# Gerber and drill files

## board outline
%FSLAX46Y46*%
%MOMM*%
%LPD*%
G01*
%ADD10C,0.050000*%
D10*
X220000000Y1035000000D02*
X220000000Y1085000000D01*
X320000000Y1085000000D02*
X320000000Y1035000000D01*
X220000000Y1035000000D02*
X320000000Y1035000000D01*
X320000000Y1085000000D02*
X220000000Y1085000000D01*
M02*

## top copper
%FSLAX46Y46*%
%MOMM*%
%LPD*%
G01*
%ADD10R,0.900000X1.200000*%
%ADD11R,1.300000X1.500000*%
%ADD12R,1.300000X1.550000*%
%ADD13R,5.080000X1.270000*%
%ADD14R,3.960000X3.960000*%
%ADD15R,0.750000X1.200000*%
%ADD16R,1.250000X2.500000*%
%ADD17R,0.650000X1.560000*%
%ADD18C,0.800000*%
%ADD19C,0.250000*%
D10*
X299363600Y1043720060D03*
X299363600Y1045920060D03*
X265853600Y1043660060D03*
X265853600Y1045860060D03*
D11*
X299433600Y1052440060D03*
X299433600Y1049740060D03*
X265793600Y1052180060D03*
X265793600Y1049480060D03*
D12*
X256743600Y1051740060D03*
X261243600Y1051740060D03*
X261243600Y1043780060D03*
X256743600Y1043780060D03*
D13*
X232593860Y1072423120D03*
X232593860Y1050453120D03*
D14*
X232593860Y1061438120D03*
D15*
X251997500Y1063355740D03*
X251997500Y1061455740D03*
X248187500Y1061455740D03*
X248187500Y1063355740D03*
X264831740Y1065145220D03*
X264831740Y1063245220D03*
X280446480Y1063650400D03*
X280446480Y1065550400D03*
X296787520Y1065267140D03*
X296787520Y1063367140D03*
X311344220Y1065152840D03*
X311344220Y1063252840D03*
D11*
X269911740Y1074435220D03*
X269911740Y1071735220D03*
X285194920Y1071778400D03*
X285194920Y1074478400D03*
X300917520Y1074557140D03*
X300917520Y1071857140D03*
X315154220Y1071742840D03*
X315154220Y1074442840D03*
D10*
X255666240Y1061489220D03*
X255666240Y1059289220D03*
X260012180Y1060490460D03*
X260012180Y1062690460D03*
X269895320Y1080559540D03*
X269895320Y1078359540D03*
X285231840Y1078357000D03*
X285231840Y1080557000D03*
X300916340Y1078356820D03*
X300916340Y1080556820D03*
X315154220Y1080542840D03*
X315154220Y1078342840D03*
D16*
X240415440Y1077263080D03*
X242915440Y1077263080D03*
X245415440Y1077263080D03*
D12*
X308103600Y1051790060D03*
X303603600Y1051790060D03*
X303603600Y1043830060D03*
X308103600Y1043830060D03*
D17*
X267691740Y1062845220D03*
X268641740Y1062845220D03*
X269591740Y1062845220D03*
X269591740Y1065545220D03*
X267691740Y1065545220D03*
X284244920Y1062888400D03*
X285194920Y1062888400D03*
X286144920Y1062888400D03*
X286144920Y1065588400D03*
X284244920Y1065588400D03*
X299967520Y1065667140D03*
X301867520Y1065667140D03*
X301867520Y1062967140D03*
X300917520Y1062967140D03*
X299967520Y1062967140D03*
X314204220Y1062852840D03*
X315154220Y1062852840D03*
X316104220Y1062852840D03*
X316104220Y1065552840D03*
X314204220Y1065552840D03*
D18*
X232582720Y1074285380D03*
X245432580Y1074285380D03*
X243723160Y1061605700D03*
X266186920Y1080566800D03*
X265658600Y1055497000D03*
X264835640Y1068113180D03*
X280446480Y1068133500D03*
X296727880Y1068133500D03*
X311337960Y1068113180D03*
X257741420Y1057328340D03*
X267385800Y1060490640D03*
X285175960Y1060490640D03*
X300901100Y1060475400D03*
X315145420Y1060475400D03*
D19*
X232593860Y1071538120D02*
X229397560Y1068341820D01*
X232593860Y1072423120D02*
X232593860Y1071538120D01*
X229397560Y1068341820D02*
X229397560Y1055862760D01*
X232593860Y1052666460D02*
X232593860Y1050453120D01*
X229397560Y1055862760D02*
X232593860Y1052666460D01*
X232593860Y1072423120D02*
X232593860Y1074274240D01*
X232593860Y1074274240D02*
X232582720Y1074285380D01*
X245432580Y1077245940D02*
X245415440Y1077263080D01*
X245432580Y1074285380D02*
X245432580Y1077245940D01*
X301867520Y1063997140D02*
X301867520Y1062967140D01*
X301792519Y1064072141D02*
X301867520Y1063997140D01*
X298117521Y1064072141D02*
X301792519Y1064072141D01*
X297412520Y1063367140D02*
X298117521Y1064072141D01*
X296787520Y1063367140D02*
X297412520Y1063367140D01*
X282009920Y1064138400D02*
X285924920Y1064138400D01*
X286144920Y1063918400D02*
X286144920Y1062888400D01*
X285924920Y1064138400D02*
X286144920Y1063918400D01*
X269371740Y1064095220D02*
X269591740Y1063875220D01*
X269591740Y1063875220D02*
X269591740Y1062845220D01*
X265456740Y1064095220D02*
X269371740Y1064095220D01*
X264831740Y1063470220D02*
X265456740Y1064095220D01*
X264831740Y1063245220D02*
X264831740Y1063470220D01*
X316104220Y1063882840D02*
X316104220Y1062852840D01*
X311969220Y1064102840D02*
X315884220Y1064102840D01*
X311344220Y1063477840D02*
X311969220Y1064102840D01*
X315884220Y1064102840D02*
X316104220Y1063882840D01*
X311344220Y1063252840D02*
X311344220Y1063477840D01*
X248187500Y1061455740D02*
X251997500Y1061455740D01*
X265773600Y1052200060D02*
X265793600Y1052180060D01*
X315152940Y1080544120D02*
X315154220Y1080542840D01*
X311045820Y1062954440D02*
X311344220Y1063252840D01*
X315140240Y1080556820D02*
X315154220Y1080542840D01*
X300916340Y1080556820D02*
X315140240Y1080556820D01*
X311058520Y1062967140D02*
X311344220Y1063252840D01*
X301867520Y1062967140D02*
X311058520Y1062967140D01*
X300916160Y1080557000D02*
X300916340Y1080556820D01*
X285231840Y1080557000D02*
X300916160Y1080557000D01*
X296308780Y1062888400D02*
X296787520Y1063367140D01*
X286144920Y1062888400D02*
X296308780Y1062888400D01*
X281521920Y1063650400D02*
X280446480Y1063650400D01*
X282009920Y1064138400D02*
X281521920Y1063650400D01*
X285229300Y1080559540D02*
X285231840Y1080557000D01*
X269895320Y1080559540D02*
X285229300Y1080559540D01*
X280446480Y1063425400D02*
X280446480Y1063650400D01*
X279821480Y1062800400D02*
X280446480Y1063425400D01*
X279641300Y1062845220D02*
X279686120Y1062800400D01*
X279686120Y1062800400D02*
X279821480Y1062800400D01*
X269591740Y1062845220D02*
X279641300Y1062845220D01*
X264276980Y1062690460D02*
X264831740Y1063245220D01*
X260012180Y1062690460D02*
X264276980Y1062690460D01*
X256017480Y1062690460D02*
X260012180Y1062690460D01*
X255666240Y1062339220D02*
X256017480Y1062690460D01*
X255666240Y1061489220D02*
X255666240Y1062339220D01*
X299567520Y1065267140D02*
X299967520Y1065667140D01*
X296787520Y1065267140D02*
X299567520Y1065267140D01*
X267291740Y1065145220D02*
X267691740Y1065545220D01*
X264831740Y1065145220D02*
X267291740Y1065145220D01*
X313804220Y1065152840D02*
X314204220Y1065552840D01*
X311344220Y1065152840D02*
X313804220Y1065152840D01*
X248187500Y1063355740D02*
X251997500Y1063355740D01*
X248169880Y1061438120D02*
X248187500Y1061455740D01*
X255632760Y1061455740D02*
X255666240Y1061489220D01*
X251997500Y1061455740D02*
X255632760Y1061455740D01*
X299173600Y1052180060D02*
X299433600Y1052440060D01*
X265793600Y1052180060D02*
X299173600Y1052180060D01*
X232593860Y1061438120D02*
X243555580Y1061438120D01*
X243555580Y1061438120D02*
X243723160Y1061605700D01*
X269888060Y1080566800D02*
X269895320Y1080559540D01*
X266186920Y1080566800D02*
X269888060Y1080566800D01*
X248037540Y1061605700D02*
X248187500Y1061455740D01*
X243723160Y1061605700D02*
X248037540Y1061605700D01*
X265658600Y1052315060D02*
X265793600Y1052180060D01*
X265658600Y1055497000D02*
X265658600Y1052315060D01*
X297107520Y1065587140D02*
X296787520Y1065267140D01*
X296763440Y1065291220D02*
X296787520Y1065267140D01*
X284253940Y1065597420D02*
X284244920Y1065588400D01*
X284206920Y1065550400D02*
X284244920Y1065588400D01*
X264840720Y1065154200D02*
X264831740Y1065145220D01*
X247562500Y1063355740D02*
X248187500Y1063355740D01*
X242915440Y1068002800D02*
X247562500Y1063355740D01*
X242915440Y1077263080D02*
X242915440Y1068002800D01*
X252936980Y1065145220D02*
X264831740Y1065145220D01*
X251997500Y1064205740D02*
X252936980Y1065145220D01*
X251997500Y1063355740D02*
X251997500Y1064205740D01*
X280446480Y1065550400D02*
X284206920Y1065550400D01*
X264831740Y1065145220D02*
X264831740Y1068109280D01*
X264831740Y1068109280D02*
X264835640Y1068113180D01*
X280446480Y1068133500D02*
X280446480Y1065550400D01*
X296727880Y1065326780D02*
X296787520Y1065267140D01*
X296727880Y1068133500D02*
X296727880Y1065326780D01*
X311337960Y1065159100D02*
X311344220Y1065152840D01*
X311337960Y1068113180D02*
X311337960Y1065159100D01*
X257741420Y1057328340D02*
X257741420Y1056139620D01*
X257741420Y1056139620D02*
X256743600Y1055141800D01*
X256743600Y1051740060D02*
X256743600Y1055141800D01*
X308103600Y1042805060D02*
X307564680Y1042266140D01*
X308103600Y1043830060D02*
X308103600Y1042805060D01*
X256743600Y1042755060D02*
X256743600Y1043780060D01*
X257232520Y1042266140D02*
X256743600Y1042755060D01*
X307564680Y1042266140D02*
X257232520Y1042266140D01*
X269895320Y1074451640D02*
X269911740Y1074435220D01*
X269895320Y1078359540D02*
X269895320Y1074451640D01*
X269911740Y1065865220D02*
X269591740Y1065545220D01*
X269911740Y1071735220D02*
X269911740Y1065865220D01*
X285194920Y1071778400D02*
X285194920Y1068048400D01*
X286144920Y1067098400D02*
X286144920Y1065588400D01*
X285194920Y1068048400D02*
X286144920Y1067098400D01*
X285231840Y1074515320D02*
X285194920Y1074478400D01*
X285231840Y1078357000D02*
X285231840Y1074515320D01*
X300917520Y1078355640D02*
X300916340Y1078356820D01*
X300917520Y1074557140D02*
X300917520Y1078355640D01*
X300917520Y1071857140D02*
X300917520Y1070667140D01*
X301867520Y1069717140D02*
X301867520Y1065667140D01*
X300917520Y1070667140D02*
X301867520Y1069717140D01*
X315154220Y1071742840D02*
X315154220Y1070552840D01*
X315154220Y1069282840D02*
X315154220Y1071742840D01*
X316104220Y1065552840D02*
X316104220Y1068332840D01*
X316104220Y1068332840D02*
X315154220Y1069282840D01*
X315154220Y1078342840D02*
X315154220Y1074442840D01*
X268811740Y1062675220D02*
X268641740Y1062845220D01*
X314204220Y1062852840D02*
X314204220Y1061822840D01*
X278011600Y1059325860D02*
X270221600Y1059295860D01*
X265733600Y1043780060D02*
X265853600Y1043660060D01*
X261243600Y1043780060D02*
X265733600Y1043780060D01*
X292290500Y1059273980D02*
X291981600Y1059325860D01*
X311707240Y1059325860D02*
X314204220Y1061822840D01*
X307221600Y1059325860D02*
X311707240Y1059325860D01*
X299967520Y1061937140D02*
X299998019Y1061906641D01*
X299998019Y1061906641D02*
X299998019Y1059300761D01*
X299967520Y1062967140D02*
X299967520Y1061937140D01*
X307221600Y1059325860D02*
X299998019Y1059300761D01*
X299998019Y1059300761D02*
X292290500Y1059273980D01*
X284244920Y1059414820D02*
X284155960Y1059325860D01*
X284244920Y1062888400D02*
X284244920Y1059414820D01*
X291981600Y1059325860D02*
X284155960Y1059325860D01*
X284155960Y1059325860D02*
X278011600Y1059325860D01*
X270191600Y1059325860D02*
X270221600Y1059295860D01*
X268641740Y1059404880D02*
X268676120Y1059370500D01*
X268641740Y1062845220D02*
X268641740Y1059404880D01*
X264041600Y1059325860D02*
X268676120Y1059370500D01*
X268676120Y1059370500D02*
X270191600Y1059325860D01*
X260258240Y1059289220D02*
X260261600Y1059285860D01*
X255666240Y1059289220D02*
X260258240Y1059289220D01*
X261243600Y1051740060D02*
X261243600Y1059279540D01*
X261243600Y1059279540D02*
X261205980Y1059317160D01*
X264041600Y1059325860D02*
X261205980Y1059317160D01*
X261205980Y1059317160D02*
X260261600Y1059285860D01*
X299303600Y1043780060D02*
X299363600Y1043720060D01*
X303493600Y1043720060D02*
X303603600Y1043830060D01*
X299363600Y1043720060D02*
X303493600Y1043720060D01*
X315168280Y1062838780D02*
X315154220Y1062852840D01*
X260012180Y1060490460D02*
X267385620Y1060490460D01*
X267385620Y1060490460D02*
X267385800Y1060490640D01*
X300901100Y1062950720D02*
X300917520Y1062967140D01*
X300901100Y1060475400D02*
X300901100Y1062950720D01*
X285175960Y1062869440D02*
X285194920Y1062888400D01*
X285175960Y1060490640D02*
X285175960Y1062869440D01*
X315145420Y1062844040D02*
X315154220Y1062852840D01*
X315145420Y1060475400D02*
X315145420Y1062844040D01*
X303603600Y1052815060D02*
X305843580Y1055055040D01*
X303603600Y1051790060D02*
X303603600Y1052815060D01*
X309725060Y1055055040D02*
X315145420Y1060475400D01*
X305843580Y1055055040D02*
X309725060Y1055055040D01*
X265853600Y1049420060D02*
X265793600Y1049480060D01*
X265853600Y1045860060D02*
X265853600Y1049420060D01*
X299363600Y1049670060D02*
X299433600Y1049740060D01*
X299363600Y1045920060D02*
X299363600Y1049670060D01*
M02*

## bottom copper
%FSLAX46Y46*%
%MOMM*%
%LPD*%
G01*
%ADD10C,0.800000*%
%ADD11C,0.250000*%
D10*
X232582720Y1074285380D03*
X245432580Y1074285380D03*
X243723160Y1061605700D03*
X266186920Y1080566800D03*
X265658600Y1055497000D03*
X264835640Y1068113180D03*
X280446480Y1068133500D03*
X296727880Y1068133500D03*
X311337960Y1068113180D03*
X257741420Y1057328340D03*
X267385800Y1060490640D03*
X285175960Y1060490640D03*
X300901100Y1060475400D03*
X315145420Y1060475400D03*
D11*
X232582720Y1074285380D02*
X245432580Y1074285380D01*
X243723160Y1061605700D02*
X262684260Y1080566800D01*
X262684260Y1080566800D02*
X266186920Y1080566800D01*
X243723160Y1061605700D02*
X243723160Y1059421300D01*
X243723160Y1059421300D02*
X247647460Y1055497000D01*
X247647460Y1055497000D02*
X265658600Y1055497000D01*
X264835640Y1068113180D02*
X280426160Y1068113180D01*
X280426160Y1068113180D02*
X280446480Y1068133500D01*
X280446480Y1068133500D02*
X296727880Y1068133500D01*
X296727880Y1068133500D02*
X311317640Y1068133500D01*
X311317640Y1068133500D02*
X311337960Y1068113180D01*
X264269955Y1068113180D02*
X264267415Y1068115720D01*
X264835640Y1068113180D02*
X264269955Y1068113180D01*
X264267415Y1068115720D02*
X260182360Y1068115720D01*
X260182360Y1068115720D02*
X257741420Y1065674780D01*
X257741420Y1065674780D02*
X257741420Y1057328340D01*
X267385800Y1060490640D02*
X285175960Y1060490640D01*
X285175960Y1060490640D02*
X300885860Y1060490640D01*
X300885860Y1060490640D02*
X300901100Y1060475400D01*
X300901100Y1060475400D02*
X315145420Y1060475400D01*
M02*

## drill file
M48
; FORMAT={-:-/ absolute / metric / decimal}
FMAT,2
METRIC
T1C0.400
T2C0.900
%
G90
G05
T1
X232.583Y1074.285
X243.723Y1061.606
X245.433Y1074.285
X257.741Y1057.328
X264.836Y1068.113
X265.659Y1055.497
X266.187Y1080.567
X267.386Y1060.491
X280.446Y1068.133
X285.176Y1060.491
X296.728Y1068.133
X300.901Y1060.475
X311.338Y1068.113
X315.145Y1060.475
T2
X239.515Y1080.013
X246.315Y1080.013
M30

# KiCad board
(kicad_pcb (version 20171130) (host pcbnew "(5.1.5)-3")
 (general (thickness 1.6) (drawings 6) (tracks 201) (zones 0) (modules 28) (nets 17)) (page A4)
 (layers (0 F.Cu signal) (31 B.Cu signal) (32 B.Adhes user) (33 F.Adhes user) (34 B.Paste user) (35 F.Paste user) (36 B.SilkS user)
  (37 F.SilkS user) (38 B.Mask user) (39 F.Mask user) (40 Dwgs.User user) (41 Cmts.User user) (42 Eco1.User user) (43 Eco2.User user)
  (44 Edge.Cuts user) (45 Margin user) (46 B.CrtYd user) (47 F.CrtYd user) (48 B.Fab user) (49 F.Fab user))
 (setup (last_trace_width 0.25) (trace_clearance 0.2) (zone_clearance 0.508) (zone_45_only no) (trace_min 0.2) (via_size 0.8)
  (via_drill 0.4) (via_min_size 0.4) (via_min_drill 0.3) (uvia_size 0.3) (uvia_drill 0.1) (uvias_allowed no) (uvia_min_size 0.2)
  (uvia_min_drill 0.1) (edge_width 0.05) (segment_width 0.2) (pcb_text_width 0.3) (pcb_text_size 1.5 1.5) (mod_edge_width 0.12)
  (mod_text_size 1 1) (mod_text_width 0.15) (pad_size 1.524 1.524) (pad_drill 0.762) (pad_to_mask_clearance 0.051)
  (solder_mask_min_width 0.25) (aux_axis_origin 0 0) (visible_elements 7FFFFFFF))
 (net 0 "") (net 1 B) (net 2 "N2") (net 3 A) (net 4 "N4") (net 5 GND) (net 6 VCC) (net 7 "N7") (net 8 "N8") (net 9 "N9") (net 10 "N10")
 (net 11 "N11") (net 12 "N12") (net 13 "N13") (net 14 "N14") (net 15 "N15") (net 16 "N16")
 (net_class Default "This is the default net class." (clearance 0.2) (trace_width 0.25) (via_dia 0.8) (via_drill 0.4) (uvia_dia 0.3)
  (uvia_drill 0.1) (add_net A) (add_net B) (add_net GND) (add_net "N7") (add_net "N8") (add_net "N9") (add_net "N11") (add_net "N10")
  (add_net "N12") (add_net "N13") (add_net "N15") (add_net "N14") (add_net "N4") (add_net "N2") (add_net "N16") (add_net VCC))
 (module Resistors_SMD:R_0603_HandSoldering (layer F.Cu) (at 299.3636 -1044.82006 90)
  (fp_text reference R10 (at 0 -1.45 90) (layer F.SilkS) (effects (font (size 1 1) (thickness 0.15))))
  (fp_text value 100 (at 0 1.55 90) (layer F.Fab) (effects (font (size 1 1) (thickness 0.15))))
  (pad 1 smd rect (at -1.1 0 90) (size 1.2 0.9) (layers F.Cu F.Paste F.Mask) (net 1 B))
  (pad 2 smd rect (at 1.1 0 90) (size 1.2 0.9) (layers F.Cu F.Paste F.Mask) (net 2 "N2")))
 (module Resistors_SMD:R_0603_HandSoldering (layer F.Cu) (at 265.8536 -1044.76006 90)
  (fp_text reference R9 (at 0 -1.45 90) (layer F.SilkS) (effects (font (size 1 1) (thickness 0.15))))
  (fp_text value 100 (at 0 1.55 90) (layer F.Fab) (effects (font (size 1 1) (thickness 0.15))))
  (pad 1 smd rect (at -1.1 0 90) (size 1.2 0.9) (layers F.Cu F.Paste F.Mask) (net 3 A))
  (pad 2 smd rect (at 1.1 0 90) (size 1.2 0.9) (layers F.Cu F.Paste F.Mask) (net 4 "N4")))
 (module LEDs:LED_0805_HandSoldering (layer F.Cu) (at 299.4336 -1051.09006 270)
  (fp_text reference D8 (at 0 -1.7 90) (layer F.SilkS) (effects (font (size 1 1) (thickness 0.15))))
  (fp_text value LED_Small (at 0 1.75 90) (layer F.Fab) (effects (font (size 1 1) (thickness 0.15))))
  (pad 1 smd rect (at -1.35 0 270) (size 1.5 1.3) (layers F.Cu F.Paste F.Mask) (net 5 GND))
  (pad 2 smd rect (at 1.35 0 270) (size 1.5 1.3) (layers F.Cu F.Paste F.Mask) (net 2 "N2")))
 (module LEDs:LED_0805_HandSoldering (layer F.Cu) (at 265.7936 -1050.83006 270)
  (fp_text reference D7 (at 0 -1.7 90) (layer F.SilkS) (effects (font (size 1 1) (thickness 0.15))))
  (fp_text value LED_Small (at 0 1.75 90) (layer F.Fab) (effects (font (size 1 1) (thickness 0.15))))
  (pad 1 smd rect (at -1.35 0 270) (size 1.5 1.3) (layers F.Cu F.Paste F.Mask) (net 5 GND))
  (pad 2 smd rect (at 1.35 0 270) (size 1.5 1.3) (layers F.Cu F.Paste F.Mask) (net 4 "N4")))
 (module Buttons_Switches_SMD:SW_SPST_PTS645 (layer F.Cu) (at 258.9936 -1047.76006 270)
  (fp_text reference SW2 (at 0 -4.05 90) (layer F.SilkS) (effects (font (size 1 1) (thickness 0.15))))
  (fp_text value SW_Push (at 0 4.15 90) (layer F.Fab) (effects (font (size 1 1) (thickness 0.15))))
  (pad 2 smd rect (at -3.98 2.25 270) (size 1.55 1.3) (layers F.Cu F.Paste F.Mask) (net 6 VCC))
  (pad 1 smd rect (at -3.98 -2.25 270) (size 1.55 1.3) (layers F.Cu F.Paste F.Mask) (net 3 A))
  (pad 1 smd rect (at 3.98 -2.25 270) (size 1.55 1.3) (layers F.Cu F.Paste F.Mask) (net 3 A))
  (pad 2 smd rect (at 3.98 2.25 270) (size 1.55 1.3) (layers F.Cu F.Paste F.Mask) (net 6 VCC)))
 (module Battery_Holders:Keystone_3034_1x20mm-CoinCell (layer F.Cu) (at 232.59386 -1061.43812 270)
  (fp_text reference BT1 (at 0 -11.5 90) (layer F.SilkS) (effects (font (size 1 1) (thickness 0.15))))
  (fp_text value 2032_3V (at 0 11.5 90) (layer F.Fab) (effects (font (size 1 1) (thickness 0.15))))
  (pad 1 smd rect (at -10.985 0 270) (size 1.27 5.08) (layers F.Cu F.Paste F.Mask) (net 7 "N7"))
  (pad 1 smd rect (at 10.985 0 270) (size 1.27 5.08) (layers F.Cu F.Paste F.Mask) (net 7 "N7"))
  (pad 2 smd rect (at 0 0 270) (size 3.96 3.96) (layers F.Cu F.Paste F.Mask) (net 5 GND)))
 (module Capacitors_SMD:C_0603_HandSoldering (layer F.Cu) (at 251.9975 -1062.40574 270)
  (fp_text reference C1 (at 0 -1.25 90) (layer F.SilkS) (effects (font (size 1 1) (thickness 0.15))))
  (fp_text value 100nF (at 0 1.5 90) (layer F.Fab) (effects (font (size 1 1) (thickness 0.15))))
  (pad 1 smd rect (at -0.95 0 270) (size 1.2 0.75) (layers F.Cu F.Paste F.Mask) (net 6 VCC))
  (pad 2 smd rect (at 0.95 0 270) (size 1.2 0.75) (layers F.Cu F.Paste F.Mask) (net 5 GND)))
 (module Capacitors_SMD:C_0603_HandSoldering (layer F.Cu) (at 248.1875 -1062.40574 270)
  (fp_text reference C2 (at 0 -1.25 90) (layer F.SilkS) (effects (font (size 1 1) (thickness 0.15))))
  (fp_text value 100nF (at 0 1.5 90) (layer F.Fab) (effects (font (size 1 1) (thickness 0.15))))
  (pad 2 smd rect (at 0.95 0 270) (size 1.2 0.75) (layers F.Cu F.Paste F.Mask) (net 5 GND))
  (pad 1 smd rect (at -0.95 0 270) (size 1.2 0.75) (layers F.Cu F.Paste F.Mask) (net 6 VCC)))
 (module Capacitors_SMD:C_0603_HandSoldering (layer F.Cu) (at 264.83174 -1064.19522 270)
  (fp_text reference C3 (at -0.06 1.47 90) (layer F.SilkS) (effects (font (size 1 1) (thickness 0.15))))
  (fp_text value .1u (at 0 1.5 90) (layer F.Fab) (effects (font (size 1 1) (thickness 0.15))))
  (pad 1 smd rect (at -0.95 0 270) (size 1.2 0.75) (layers F.Cu F.Paste F.Mask) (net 6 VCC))
  (pad 2 smd rect (at 0.95 0 270) (size 1.2 0.75) (layers F.Cu F.Paste F.Mask) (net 5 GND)))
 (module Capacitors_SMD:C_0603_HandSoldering (layer F.Cu) (at 280.44648 -1064.6004 270)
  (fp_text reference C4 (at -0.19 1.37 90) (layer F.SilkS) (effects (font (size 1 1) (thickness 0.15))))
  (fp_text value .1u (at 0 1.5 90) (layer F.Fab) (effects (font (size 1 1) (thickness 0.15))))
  (pad 2 smd rect (at 0.95 0 270) (size 1.2 0.75) (layers F.Cu F.Paste F.Mask) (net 5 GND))
  (pad 1 smd rect (at -0.95 0 270) (size 1.2 0.75) (layers F.Cu F.Paste F.Mask) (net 6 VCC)))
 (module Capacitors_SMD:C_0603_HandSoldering (layer F.Cu) (at 296.78752 -1064.31714 270)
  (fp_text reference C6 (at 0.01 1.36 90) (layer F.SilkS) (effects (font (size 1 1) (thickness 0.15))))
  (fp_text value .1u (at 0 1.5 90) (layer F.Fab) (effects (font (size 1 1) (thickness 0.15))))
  (pad 1 smd rect (at -0.95 0 270) (size 1.2 0.75) (layers F.Cu F.Paste F.Mask) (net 6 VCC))
  (pad 2 smd rect (at 0.95 0 270) (size 1.2 0.75) (layers F.Cu F.Paste F.Mask) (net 5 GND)))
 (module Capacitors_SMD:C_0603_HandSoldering (layer F.Cu) (at 311.34422 -1064.20284 270)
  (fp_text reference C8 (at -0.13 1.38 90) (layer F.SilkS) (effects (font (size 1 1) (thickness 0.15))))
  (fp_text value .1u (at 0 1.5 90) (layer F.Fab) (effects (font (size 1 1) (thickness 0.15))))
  (pad 1 smd rect (at -0.95 0 270) (size 1.2 0.75) (layers F.Cu F.Paste F.Mask) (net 6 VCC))
  (pad 2 smd rect (at 0.95 0 270) (size 1.2 0.75) (layers F.Cu F.Paste F.Mask) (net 5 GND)))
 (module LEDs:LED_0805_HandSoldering (layer F.Cu) (at 269.91174 -1073.08522 270)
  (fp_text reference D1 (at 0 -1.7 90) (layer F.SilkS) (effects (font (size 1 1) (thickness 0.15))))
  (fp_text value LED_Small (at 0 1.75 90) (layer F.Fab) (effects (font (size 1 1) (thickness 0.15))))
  (pad 1 smd rect (at -1.35 0 270) (size 1.5 1.3) (layers F.Cu F.Paste F.Mask) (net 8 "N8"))
  (pad 2 smd rect (at 1.35 0 270) (size 1.5 1.3) (layers F.Cu F.Paste F.Mask) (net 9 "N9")))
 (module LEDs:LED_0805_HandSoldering (layer F.Cu) (at 285.19492 -1073.1284 270)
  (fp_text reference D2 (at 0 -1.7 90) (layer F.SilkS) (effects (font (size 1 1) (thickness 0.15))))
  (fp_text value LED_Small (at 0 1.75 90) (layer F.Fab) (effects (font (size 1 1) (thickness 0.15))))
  (pad 2 smd rect (at 1.35 0 270) (size 1.5 1.3) (layers F.Cu F.Paste F.Mask) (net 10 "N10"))
  (pad 1 smd rect (at -1.35 0 270) (size 1.5 1.3) (layers F.Cu F.Paste F.Mask) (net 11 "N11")))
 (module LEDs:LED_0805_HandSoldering (layer F.Cu) (at 300.91752 -1073.20714 270)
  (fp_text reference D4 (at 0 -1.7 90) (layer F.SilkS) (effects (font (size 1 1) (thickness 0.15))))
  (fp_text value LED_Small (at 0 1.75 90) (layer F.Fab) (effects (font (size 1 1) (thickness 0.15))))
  (pad 1 smd rect (at -1.35 0 270) (size 1.5 1.3) (layers F.Cu F.Paste F.Mask) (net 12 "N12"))
  (pad 2 smd rect (at 1.35 0 270) (size 1.5 1.3) (layers F.Cu F.Paste F.Mask) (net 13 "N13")))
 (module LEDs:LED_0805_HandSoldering (layer F.Cu) (at 315.15422 -1073.09284 270)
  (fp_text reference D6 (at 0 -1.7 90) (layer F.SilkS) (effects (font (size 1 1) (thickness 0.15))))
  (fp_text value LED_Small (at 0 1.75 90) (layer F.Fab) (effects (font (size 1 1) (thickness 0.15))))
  (pad 2 smd rect (at 1.35 0 270) (size 1.5 1.3) (layers F.Cu F.Paste F.Mask) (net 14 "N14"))
  (pad 1 smd rect (at -1.35 0 270) (size 1.5 1.3) (layers F.Cu F.Paste F.Mask) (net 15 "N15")))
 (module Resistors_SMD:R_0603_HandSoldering (layer F.Cu) (at 255.66624 -1060.38922 270)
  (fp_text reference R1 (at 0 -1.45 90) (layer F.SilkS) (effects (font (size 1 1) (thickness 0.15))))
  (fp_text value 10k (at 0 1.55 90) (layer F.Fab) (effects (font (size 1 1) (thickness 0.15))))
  (pad 1 smd rect (at -1.1 0 270) (size 1.2 0.9) (layers F.Cu F.Paste F.Mask) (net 5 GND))
  (pad 2 smd rect (at 1.1 0 270) (size 1.2 0.9) (layers F.Cu F.Paste F.Mask) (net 3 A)))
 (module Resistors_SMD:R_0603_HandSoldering (layer F.Cu) (at 260.01218 -1061.59046 90)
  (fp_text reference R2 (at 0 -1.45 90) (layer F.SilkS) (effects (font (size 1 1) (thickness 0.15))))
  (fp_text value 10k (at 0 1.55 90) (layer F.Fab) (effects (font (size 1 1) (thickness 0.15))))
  (pad 1 smd rect (at -1.1 0 90) (size 1.2 0.9) (layers F.Cu F.Paste F.Mask) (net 1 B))
  (pad 2 smd rect (at 1.1 0 90) (size 1.2 0.9) (layers F.Cu F.Paste F.Mask) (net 5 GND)))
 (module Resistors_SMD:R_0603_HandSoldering (layer F.Cu) (at 269.89532 -1079.45954 270)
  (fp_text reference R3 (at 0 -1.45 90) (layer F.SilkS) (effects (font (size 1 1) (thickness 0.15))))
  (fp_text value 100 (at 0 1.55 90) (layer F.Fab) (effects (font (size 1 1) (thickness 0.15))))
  (pad 1 smd rect (at -1.1 0 270) (size 1.2 0.9) (layers F.Cu F.Paste F.Mask) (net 5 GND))
  (pad 2 smd rect (at 1.1 0 270) (size 1.2 0.9) (layers F.Cu F.Paste F.Mask) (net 8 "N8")))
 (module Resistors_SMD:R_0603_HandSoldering (layer F.Cu) (at 285.23184 -1079.457 270)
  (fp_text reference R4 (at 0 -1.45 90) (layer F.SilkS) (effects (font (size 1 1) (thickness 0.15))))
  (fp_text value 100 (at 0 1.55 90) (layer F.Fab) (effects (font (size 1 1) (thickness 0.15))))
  (pad 2 smd rect (at 1.1 0 270) (size 1.2 0.9) (layers F.Cu F.Paste F.Mask) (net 11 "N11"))
  (pad 1 smd rect (at -1.1 0 270) (size 1.2 0.9) (layers F.Cu F.Paste F.Mask) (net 5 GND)))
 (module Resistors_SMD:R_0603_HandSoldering (layer F.Cu) (at 300.91634 -1079.45682 270)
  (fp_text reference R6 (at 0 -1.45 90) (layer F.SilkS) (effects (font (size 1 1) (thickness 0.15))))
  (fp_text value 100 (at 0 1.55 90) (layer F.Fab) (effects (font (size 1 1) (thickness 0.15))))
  (pad 2 smd rect (at 1.1 0 270) (size 1.2 0.9) (layers F.Cu F.Paste F.Mask) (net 12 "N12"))
  (pad 1 smd rect (at -1.1 0 270) (size 1.2 0.9) (layers F.Cu F.Paste F.Mask) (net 5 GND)))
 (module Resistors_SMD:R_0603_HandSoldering (layer F.Cu) (at 315.15422 -1079.44284 270)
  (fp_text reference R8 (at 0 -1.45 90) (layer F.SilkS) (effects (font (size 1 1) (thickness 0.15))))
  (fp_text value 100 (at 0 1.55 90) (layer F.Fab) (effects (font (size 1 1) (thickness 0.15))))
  (pad 1 smd rect (at -1.1 0 270) (size 1.2 0.9) (layers F.Cu F.Paste F.Mask) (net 5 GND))
  (pad 2 smd rect (at 1.1 0 270) (size 1.2 0.9) (layers F.Cu F.Paste F.Mask) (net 15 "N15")))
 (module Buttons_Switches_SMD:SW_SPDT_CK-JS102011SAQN (layer F.Cu) (at 242.91544 -1080.01308 180)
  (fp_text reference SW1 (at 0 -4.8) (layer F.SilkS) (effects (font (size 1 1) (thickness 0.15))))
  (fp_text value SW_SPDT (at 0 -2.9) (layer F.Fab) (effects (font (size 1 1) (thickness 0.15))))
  (pad "" np_thru_hole circle (at 3.4 0 180) (size 0.9 0.9) (drill 0.9) (layers *.Cu *.Mask))
  (pad "" np_thru_hole circle (at -3.4 0 180) (size 0.9 0.9) (drill 0.9) (layers *.Cu *.Mask))
  (pad 3 smd rect (at 2.5 -2.75 180) (size 1.25 2.5) (layers F.Cu F.Paste F.Mask) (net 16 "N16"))
  (pad 2 smd rect (at 0 -2.75 180) (size 1.25 2.5) (layers F.Cu F.Paste F.Mask) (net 6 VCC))
  (pad 1 smd rect (at -2.5 -2.75 180) (size 1.25 2.5) (layers F.Cu F.Paste F.Mask) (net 7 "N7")))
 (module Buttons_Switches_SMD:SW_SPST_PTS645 (layer F.Cu) (at 305.8536 -1047.81006 90)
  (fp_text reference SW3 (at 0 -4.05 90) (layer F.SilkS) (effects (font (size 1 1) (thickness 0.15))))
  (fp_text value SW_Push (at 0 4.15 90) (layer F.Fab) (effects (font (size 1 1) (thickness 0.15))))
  (pad 2 smd rect (at 3.98 2.25 90) (size 1.55 1.3) (layers F.Cu F.Paste F.Mask) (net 6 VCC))
  (pad 1 smd rect (at 3.98 -2.25 90) (size 1.55 1.3) (layers F.Cu F.Paste F.Mask) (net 1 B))
  (pad 1 smd rect (at -3.98 -2.25 90) (size 1.55 1.3) (layers F.Cu F.Paste F.Mask) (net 1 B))
  (pad 2 smd rect (at -3.98 2.25 90) (size 1.55 1.3) (layers F.Cu F.Paste F.Mask) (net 6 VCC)))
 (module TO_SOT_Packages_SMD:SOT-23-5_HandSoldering (layer F.Cu) (at 268.64174 -1064.19522 90)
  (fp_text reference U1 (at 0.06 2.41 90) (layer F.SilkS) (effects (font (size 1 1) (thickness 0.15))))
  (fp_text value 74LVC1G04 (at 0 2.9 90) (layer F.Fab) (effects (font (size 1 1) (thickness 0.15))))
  (pad 1 smd rect (at -1.35 -0.95 90) (size 1.56 0.65) (layers F.Cu F.Paste F.Mask))
  (pad 2 smd rect (at -1.35 0 90) (size 1.56 0.65) (layers F.Cu F.Paste F.Mask) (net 3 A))
  (pad 3 smd rect (at -1.35 0.95 90) (size 1.56 0.65) (layers F.Cu F.Paste F.Mask) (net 5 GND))
  (pad 4 smd rect (at 1.35 0.95 90) (size 1.56 0.65) (layers F.Cu F.Paste F.Mask) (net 9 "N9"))
  (pad 5 smd rect (at 1.35 -0.95 90) (size 1.56 0.65) (layers F.Cu F.Paste F.Mask) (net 6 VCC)))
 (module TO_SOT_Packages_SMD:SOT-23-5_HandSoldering (layer F.Cu) (at 285.19492 -1064.2384 90)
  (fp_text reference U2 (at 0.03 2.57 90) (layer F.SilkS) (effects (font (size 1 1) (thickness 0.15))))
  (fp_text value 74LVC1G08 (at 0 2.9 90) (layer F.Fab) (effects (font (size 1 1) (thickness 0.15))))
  (pad 1 smd rect (at -1.35 -0.95 90) (size 1.56 0.65) (layers F.Cu F.Paste F.Mask) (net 3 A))
  (pad 2 smd rect (at -1.35 0 90) (size 1.56 0.65) (layers F.Cu F.Paste F.Mask) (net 1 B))
  (pad 3 smd rect (at -1.35 0.95 90) (size 1.56 0.65) (layers F.Cu F.Paste F.Mask) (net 5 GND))
  (pad 4 smd rect (at 1.35 0.95 90) (size 1.56 0.65) (layers F.Cu F.Paste F.Mask) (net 10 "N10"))
  (pad 5 smd rect (at 1.35 -0.95 90) (size 1.56 0.65) (layers F.Cu F.Paste F.Mask) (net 6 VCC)))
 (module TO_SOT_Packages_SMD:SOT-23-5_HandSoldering (layer F.Cu) (at 300.91752 -1064.31714 90)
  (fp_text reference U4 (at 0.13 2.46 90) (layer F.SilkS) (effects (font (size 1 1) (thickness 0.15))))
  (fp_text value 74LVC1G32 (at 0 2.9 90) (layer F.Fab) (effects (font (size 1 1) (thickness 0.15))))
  (pad 5 smd rect (at 1.35 -0.95 90) (size 1.56 0.65) (layers F.Cu F.Paste F.Mask) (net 6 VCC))
  (pad 4 smd rect (at 1.35 0.95 90) (size 1.56 0.65) (layers F.Cu F.Paste F.Mask) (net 13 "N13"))
  (pad 3 smd rect (at -1.35 0.95 90) (size 1.56 0.65) (layers F.Cu F.Paste F.Mask) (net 5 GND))
  (pad 2 smd rect (at -1.35 0 90) (size 1.56 0.65) (layers F.Cu F.Paste F.Mask) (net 1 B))
  (pad 1 smd rect (at -1.35 -0.95 90) (size 1.56 0.65) (layers F.Cu F.Paste F.Mask) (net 3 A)))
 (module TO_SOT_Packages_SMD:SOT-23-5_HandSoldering (layer F.Cu) (at 315.15422 -1064.20284 90)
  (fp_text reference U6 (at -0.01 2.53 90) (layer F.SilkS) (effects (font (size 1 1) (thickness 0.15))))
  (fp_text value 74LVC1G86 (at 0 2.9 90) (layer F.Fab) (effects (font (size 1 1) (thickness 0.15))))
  (pad 1 smd rect (at -1.35 -0.95 90) (size 1.56 0.65) (layers F.Cu F.Paste F.Mask) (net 3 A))
  (pad 2 smd rect (at -1.35 0 90) (size 1.56 0.65) (layers F.Cu F.Paste F.Mask) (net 1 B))
  (pad 3 smd rect (at -1.35 0.95 90) (size 1.56 0.65) (layers F.Cu F.Paste F.Mask) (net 5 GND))
  (pad 4 smd rect (at 1.35 0.95 90) (size 1.56 0.65) (layers F.Cu F.Paste F.Mask) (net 14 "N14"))
  (pad 5 smd rect (at 1.35 -0.95 90) (size 1.56 0.65) (layers F.Cu F.Paste F.Mask) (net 6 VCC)))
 (gr_line (start 220 -1035) (end 220 -1085) (layer Edge.Cuts) (width 0.05))
 (gr_line (start 320 -1085) (end 320 -1035) (layer Edge.Cuts) (width 0.05))
 (gr_line (start 220 -1035) (end 320 -1035) (layer Edge.Cuts) (width 0.05))
 (gr_line (start 320 -1085) (end 220 -1085) (layer Edge.Cuts) (width 0.05))
 (segment (start 232.59386 -1071.53812) (end 229.39756 -1068.34182) (width 0.25) (layer F.Cu) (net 7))
 (segment (start 232.59386 -1072.42312) (end 232.59386 -1071.53812) (width 0.25) (layer F.Cu) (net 7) (status 10))
 (segment (start 229.39756 -1068.34182) (end 229.39756 -1055.86276) (width 0.25) (layer F.Cu) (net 7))
 (segment (start 232.59386 -1052.66646) (end 232.59386 -1050.45312) (width 0.25) (layer F.Cu) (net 7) (status 20))
 (segment (start 229.39756 -1055.86276) (end 232.59386 -1052.66646) (width 0.25) (layer F.Cu) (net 7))
 (via (at 232.58272 -1074.28538) (size 0.8) (drill 0.4) (layers F.Cu B.Cu) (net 7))
 (segment (start 232.59386 -1072.42312) (end 232.59386 -1074.27424) (width 0.25) (layer F.Cu) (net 7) (status 10))
 (segment (start 232.59386 -1074.27424) (end 232.58272 -1074.28538) (width 0.25) (layer F.Cu) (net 7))
 (via (at 245.43258 -1074.28538) (size 0.8) (drill 0.4) (layers F.Cu B.Cu) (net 7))
 (segment (start 232.58272 -1074.28538) (end 245.43258 -1074.28538) (width 0.25) (layer B.Cu) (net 7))
 (segment (start 245.43258 -1077.24594) (end 245.41544 -1077.26308) (width 0.25) (layer F.Cu) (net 7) (status 30))
 (segment (start 245.43258 -1074.28538) (end 245.43258 -1077.24594) (width 0.25) (layer F.Cu) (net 7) (status 20))
 (segment (start 301.86752 -1063.99714) (end 301.86752 -1062.96714) (width 0.25) (layer F.Cu) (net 5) (status 20))
 (segment (start 301.792519 -1064.072141) (end 301.86752 -1063.99714) (width 0.25) (layer F.Cu) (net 5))
 (segment (start 298.117521 -1064.072141) (end 301.792519 -1064.072141) (width 0.25) (layer F.Cu) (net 5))
 (segment (start 297.41252 -1063.36714) (end 298.117521 -1064.072141) (width 0.25) (layer F.Cu) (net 5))
 (segment (start 296.78752 -1063.36714) (end 297.41252 -1063.36714) (width 0.25) (layer F.Cu) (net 5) (status 10))
 (segment (start 282.00992 -1064.1384) (end 285.92492 -1064.1384) (width 0.25) (layer F.Cu) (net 5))
 (segment (start 286.14492 -1063.9184) (end 286.14492 -1062.8884) (width 0.25) (layer F.Cu) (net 5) (status 20))
 (segment (start 285.92492 -1064.1384) (end 286.14492 -1063.9184) (width 0.25) (layer F.Cu) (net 5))
 (segment (start 269.37174 -1064.09522) (end 269.59174 -1063.87522) (width 0.25) (layer F.Cu) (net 5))
 (segment (start 269.59174 -1063.87522) (end 269.59174 -1062.84522) (width 0.25) (layer F.Cu) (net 5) (status 20))
 (segment (start 265.45674 -1064.09522) (end 269.37174 -1064.09522) (width 0.25) (layer F.Cu) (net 5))
 (segment (start 264.83174 -1063.47022) (end 265.45674 -1064.09522) (width 0.25) (layer F.Cu) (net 5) (status 10))
 (segment (start 264.83174 -1063.24522) (end 264.83174 -1063.47022) (width 0.25) (layer F.Cu) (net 5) (status 30))
 (segment (start 316.10422 -1063.88284) (end 316.10422 -1062.85284) (width 0.25) (layer F.Cu) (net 5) (status 20))
 (segment (start 311.96922 -1064.10284) (end 315.88422 -1064.10284) (width 0.25) (layer F.Cu) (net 5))
 (segment (start 311.34422 -1063.47784) (end 311.96922 -1064.10284) (width 0.25) (layer F.Cu) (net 5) (status 10))
 (segment (start 315.88422 -1064.10284) (end 316.10422 -1063.88284) (width 0.25) (layer F.Cu) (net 5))
 (segment (start 311.34422 -1063.25284) (end 311.34422 -1063.47784) (width 0.25) (layer F.Cu) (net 5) (status 30))
 (segment (start 248.1875 -1061.45574) (end 251.9975 -1061.45574) (width 0.25) (layer F.Cu) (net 5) (status 30))
 (segment (start 265.7736 -1052.20006) (end 265.7936 -1052.18006) (width 0.25) (layer F.Cu) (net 5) (status 30))
 (segment (start 315.15294 -1080.54412) (end 315.15422 -1080.54284) (width 0.25) (layer F.Cu) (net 5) (status 30))
 (segment (start 311.04582 -1062.95444) (end 311.34422 -1063.25284) (width 0.25) (layer F.Cu) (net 5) (status 30))
 (segment (start 315.14024 -1080.55682) (end 315.15422 -1080.54284) (width 0.25) (layer F.Cu) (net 5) (status 30))
 (segment (start 300.91634 -1080.55682) (end 315.14024 -1080.55682) (width 0.25) (layer F.Cu) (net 5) (status 30))
 (segment (start 311.05852 -1062.96714) (end 311.34422 -1063.25284) (width 0.25) (layer F.Cu) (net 5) (status 30))
 (segment (start 301.86752 -1062.96714) (end 311.05852 -1062.96714) (width 0.25) (layer F.Cu) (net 5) (status 30))
 (segment (start 300.91616 -1080.557) (end 300.91634 -1080.55682) (width 0.25) (layer F.Cu) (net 5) (status 30))
 (segment (start 285.23184 -1080.557) (end 300.91616 -1080.557) (width 0.25) (layer F.Cu) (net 5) (status 30))
 (segment (start 296.30878 -1062.8884) (end 296.78752 -1063.36714) (width 0.25) (layer F.Cu) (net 5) (status 20))
 (segment (start 286.14492 -1062.8884) (end 296.30878 -1062.8884) (width 0.25) (layer F.Cu) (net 5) (status 10))
 (segment (start 281.52192 -1063.6504) (end 280.44648 -1063.6504) (width 0.25) (layer F.Cu) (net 5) (status 20))
 (segment (start 282.00992 -1064.1384) (end 281.52192 -1063.6504) (width 0.25) (layer F.Cu) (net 5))
 (segment (start 285.2293 -1080.55954) (end 285.23184 -1080.557) (width 0.25) (layer F.Cu) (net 5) (status 30))
 (segment (start 269.89532 -1080.55954) (end 285.2293 -1080.55954) (width 0.25) (layer F.Cu) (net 5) (status 30))
 (segment (start 280.44648 -1063.4254) (end 280.44648 -1063.6504) (width 0.25) (layer F.Cu) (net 5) (status 30))
 (segment (start 279.82148 -1062.8004) (end 280.44648 -1063.4254) (width 0.25) (layer F.Cu) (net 5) (status 20))
 (segment (start 279.6413 -1062.84522) (end 279.68612 -1062.8004) (width 0.25) (layer F.Cu) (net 5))
 (segment (start 279.68612 -1062.8004) (end 279.82148 -1062.8004) (width 0.25) (layer F.Cu) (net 5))
 (segment (start 269.59174 -1062.84522) (end 279.6413 -1062.84522) (width 0.25) (layer F.Cu) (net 5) (status 10))
 (segment (start 264.27698 -1062.69046) (end 264.83174 -1063.24522) (width 0.25) (layer F.Cu) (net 5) (status 20))
 (segment (start 260.01218 -1062.69046) (end 264.27698 -1062.69046) (width 0.25) (layer F.Cu) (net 5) (status 10))
 (segment (start 256.01748 -1062.69046) (end 260.01218 -1062.69046) (width 0.25) (layer F.Cu) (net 5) (status 20))
 (segment (start 255.66624 -1062.33922) (end 256.01748 -1062.69046) (width 0.25) (layer F.Cu) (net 5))
 (segment (start 255.66624 -1061.48922) (end 255.66624 -1062.33922) (width 0.25) (layer F.Cu) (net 5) (status 10))
 (segment (start 299.56752 -1065.26714) (end 299.96752 -1065.66714) (width 0.25) (layer F.Cu) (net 6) (status 20))
 (segment (start 296.78752 -1065.26714) (end 299.56752 -1065.26714) (width 0.25) (layer F.Cu) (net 6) (status 10))
 (segment (start 267.29174 -1065.14522) (end 267.69174 -1065.54522) (width 0.25) (layer F.Cu) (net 6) (status 20))
 (segment (start 264.83174 -1065.14522) (end 267.29174 -1065.14522) (width 0.25) (layer F.Cu) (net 6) (status 10))
 (segment (start 313.80422 -1065.15284) (end 314.20422 -1065.55284) (width 0.25) (layer F.Cu) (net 6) (status 20))
 (segment (start 311.34422 -1065.15284) (end 313.80422 -1065.15284) (width 0.25) (layer F.Cu) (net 6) (status 10))
 (segment (start 248.1875 -1063.35574) (end 251.9975 -1063.35574) (width 0.25) (layer F.Cu) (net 6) (status 30))
 (segment (start 248.16988 -1061.43812) (end 248.1875 -1061.45574) (width 0.25) (layer F.Cu) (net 5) (status 30))
 (segment (start 255.63276 -1061.45574) (end 255.66624 -1061.48922) (width 0.25) (layer F.Cu) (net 5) (status 30))
 (segment (start 251.9975 -1061.45574) (end 255.63276 -1061.45574) (width 0.25) (layer F.Cu) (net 5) (status 30))
 (segment (start 299.1736 -1052.18006) (end 299.4336 -1052.44006) (width 0.25) (layer F.Cu) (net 5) (status 30))
 (segment (start 265.7936 -1052.18006) (end 299.1736 -1052.18006) (width 0.25) (layer F.Cu) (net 5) (status 30))
 (segment (start 232.59386 -1061.43812) (end 243.55558 -1061.43812) (width 0.25) (layer F.Cu) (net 5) (status 10))
 (via (at 243.72316 -1061.6057) (size 0.8) (drill 0.4) (layers F.Cu B.Cu) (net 5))
 (segment (start 243.55558 -1061.43812) (end 243.72316 -1061.6057) (width 0.25) (layer F.Cu) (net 5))
 (via (at 266.18692 -1080.5668) (size 0.8) (drill 0.4) (layers F.Cu B.Cu) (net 5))
 (segment (start 243.72316 -1061.6057) (end 262.68426 -1080.5668) (width 0.25) (layer B.Cu) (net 5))
 (segment (start 262.68426 -1080.5668) (end 266.18692 -1080.5668) (width 0.25) (layer B.Cu) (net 5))
 (segment (start 269.88806 -1080.5668) (end 269.89532 -1080.55954) (width 0.25) (layer F.Cu) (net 5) (status 30))
 (segment (start 266.18692 -1080.5668) (end 269.88806 -1080.5668) (width 0.25) (layer F.Cu) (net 5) (status 20))
 (segment (start 248.03754 -1061.6057) (end 248.1875 -1061.45574) (width 0.25) (layer F.Cu) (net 5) (status 30))
 (segment (start 243.72316 -1061.6057) (end 248.03754 -1061.6057) (width 0.25) (layer F.Cu) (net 5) (status 20))
 (segment (start 243.72316 -1061.6057) (end 243.72316 -1059.4213) (width 0.25) (layer B.Cu) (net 5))
 (via (at 265.6586 -1055.497) (size 0.8) (drill 0.4) (layers F.Cu B.Cu) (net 5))
 (segment (start 243.72316 -1059.4213) (end 247.64746 -1055.497) (width 0.25) (layer B.Cu) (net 5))
 (segment (start 247.64746 -1055.497) (end 265.6586 -1055.497) (width 0.25) (layer B.Cu) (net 5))
 (segment (start 265.6586 -1052.31506) (end 265.7936 -1052.18006) (width 0.25) (layer F.Cu) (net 5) (status 30))
 (segment (start 265.6586 -1055.497) (end 265.6586 -1052.31506) (width 0.25) (layer F.Cu) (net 5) (status 20))
 (segment (start 297.10752 -1065.58714) (end 296.78752 -1065.26714) (width 0.25) (layer F.Cu) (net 6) (status 30))
 (segment (start 296.76344 -1065.29122) (end 296.78752 -1065.26714) (width 0.25) (layer F.Cu) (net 6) (status 30))
 (segment (start 284.25394 -1065.59742) (end 284.24492 -1065.5884) (width 0.25) (layer F.Cu) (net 6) (status 30))
 (segment (start 284.20692 -1065.5504) (end 284.24492 -1065.5884) (width 0.25) (layer F.Cu) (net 6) (status 30))
 (segment (start 264.84072 -1065.1542) (end 264.83174 -1065.14522) (width 0.25) (layer F.Cu) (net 6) (status 30))
 (segment (start 247.5625 -1063.35574) (end 248.1875 -1063.35574) (width 0.25) (layer F.Cu) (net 6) (status 20))
 (segment (start 242.91544 -1068.0028) (end 247.5625 -1063.35574) (width 0.25) (layer F.Cu) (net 6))
 (segment (start 242.91544 -1077.26308) (end 242.91544 -1068.0028) (width 0.25) (layer F.Cu) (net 6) (status 10))
 (segment (start 252.93698 -1065.14522) (end 264.83174 -1065.14522) (width 0.25) (layer F.Cu) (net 6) (status 20))
 (segment (start 251.9975 -1064.20574) (end 252.93698 -1065.14522) (width 0.25) (layer F.Cu) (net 6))
 (segment (start 251.9975 -1063.35574) (end 251.9975 -1064.20574) (width 0.25) (layer F.Cu) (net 6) (status 10))
 (segment (start 280.44648 -1065.5504) (end 284.20692 -1065.5504) (width 0.25) (layer F.Cu) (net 6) (status 30))
 (via (at 264.83564 -1068.11318) (size 0.8) (drill 0.4) (layers F.Cu B.Cu) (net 6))
 (segment (start 264.83174 -1065.14522) (end 264.83174 -1068.10928) (width 0.25) (layer F.Cu) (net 6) (status 10))
 (segment (start 264.83174 -1068.10928) (end 264.83564 -1068.11318) (width 0.25) (layer F.Cu) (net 6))
 (via (at 280.44648 -1068.1335) (size 0.8) (drill 0.4) (layers F.Cu B.Cu) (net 6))
 (segment (start 264.83564 -1068.11318) (end 280.42616 -1068.11318) (width 0.25) (layer B.Cu) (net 6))
 (segment (start 280.42616 -1068.11318) (end 280.44648 -1068.1335) (width 0.25) (layer B.Cu) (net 6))
 (segment (start 280.44648 -1068.1335) (end 280.44648 -1065.5504) (width 0.25) (layer F.Cu) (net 6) (status 20))
 (via (at 296.72788 -1068.1335) (size 0.8) (drill 0.4) (layers F.Cu B.Cu) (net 6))
 (segment (start 280.44648 -1068.1335) (end 296.72788 -1068.1335) (width 0.25) (layer B.Cu) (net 6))
 (segment (start 296.72788 -1065.32678) (end 296.78752 -1065.26714) (width 0.25) (layer F.Cu) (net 6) (status 30))
 (segment (start 296.72788 -1068.1335) (end 296.72788 -1065.32678) (width 0.25) (layer F.Cu) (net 6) (status 20))
 (via (at 311.33796 -1068.11318) (size 0.8) (drill 0.4) (layers F.Cu B.Cu) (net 6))
 (segment (start 296.72788 -1068.1335) (end 311.31764 -1068.1335) (width 0.25) (layer B.Cu) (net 6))
 (segment (start 311.31764 -1068.1335) (end 311.33796 -1068.11318) (width 0.25) (layer B.Cu) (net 6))
 (segment (start 311.33796 -1065.1591) (end 311.34422 -1065.15284) (width 0.25) (layer F.Cu) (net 6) (status 30))
 (segment (start 311.33796 -1068.11318) (end 311.33796 -1065.1591) (width 0.25) (layer F.Cu) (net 6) (status 20))
 (segment (start 264.269955 -1068.11318) (end 264.267415 -1068.11572) (width 0.25) (layer B.Cu) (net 6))
 (segment (start 264.83564 -1068.11318) (end 264.269955 -1068.11318) (width 0.25) (layer B.Cu) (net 6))
 (segment (start 264.267415 -1068.11572) (end 260.18236 -1068.11572) (width 0.25) (layer B.Cu) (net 6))
 (via (at 257.74142 -1057.32834) (size 0.8) (drill 0.4) (layers F.Cu B.Cu) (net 6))
 (segment (start 260.18236 -1068.11572) (end 257.74142 -1065.67478) (width 0.25) (layer B.Cu) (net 6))
 (segment (start 257.74142 -1065.67478) (end 257.74142 -1057.32834) (width 0.25) (layer B.Cu) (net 6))
 (segment (start 257.74142 -1057.32834) (end 257.74142 -1056.13962) (width 0.25) (layer F.Cu) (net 6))
 (segment (start 257.74142 -1056.13962) (end 256.7436 -1055.1418) (width 0.25) (layer F.Cu) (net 6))
 (segment (start 256.7436 -1051.74006) (end 256.7436 -1055.1418) (width 0.25) (layer F.Cu) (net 6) (status 10))
 (segment (start 308.1036 -1042.80506) (end 307.56468 -1042.26614) (width 0.25) (layer F.Cu) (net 6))
 (segment (start 308.1036 -1043.83006) (end 308.1036 -1042.80506) (width 0.25) (layer F.Cu) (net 6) (status 10))
 (segment (start 256.7436 -1042.75506) (end 256.7436 -1043.78006) (width 0.25) (layer F.Cu) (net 6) (status 20))
 (segment (start 257.23252 -1042.26614) (end 256.7436 -1042.75506) (width 0.25) (layer F.Cu) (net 6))
 (segment (start 307.56468 -1042.26614) (end 257.23252 -1042.26614) (width 0.25) (layer F.Cu) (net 6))
 (segment (start 269.89532 -1074.45164) (end 269.91174 -1074.43522) (width 0.25) (layer F.Cu) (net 8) (status 30))
 (segment (start 269.89532 -1078.35954) (end 269.89532 -1074.45164) (width 0.25) (layer F.Cu) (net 8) (status 30))
 (segment (start 269.91174 -1065.86522) (end 269.59174 -1065.54522) (width 0.25) (layer F.Cu) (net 9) (status 30))
 (segment (start 269.91174 -1071.73522) (end 269.91174 -1065.86522) (width 0.25) (layer F.Cu) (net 9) (status 30))
 (segment (start 285.19492 -1071.7784) (end 285.19492 -1068.0484) (width 0.25) (layer F.Cu) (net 10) (status 10))
 (segment (start 286.14492 -1067.0984) (end 286.14492 -1065.5884) (width 0.25) (layer F.Cu) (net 10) (status 20))
 (segment (start 285.19492 -1068.0484) (end 286.14492 -1067.0984) (width 0.25) (layer F.Cu) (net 10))
 (segment (start 285.23184 -1074.51532) (end 285.19492 -1074.4784) (width 0.25) (layer F.Cu) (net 11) (status 30))
 (segment (start 285.23184 -1078.357) (end 285.23184 -1074.51532) (width 0.25) (layer F.Cu) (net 11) (status 30))
 (segment (start 300.91752 -1078.35564) (end 300.91634 -1078.35682) (width 0.25) (layer F.Cu) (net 12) (status 30))
 (segment (start 300.91752 -1074.55714) (end 300.91752 -1078.35564) (width 0.25) (layer F.Cu) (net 12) (status 30))
 (segment (start 300.91752 -1071.85714) (end 300.91752 -1070.66714) (width 0.25) (layer F.Cu) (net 13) (status 10))
 (segment (start 301.86752 -1069.71714) (end 301.86752 -1065.66714) (width 0.25) (layer F.Cu) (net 13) (status 20))
 (segment (start 300.91752 -1070.66714) (end 301.86752 -1069.71714) (width 0.25) (layer F.Cu) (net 13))
 (segment (start 315.15422 -1071.74284) (end 315.15422 -1070.55284) (width 0.25) (layer F.Cu) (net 14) (status 10))
 (segment (start 315.15422 -1069.28284) (end 315.15422 -1071.74284) (width 0.25) (layer F.Cu) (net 14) (status 20))
 (segment (start 316.10422 -1065.55284) (end 316.10422 -1068.33284) (width 0.25) (layer F.Cu) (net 14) (status 10))
 (segment (start 316.10422 -1068.33284) (end 315.15422 -1069.28284) (width 0.25) (layer F.Cu) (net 14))
 (segment (start 315.15422 -1078.34284) (end 315.15422 -1074.44284) (width 0.25) (layer F.Cu) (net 15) (status 30))
 (segment (start 268.81174 -1062.67522) (end 268.64174 -1062.84522) (width 0.25) (layer F.Cu) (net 3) (status 30))
 (segment (start 314.20422 -1062.85284) (end 314.20422 -1061.82284) (width 0.25) (layer F.Cu) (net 3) (status 10))
 (segment (start 278.0116 -1059.32586) (end 270.2216 -1059.29586) (width 0.25) (layer F.Cu) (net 3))
 (segment (start 265.7336 -1043.78006) (end 265.8536 -1043.66006) (width 0.25) (layer F.Cu) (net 3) (status 30))
 (segment (start 261.2436 -1043.78006) (end 265.7336 -1043.78006) (width 0.25) (layer F.Cu) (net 3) (status 30))
 (segment (start 292.2905 -1059.27398) (end 291.9816 -1059.32586) (width 0.25) (layer F.Cu) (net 3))
 (segment (start 311.70724 -1059.32586) (end 314.20422 -1061.82284) (width 0.25) (layer F.Cu) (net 3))
 (segment (start 307.2216 -1059.32586) (end 311.70724 -1059.32586) (width 0.25) (layer F.Cu) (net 3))
 (segment (start 299.96752 -1061.93714) (end 299.998019 -1061.906641) (width 0.25) (layer F.Cu) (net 3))
 (segment (start 299.998019 -1061.906641) (end 299.998019 -1059.300761) (width 0.25) (layer F.Cu) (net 3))
 (segment (start 299.96752 -1062.96714) (end 299.96752 -1061.93714) (width 0.25) (layer F.Cu) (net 3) (status 10))
 (segment (start 307.2216 -1059.32586) (end 299.998019 -1059.300761) (width 0.25) (layer F.Cu) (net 3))
 (segment (start 299.998019 -1059.300761) (end 292.2905 -1059.27398) (width 0.25) (layer F.Cu) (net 3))
 (segment (start 284.24492 -1059.41482) (end 284.15596 -1059.32586) (width 0.25) (layer F.Cu) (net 3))
 (segment (start 284.24492 -1062.8884) (end 284.24492 -1059.41482) (width 0.25) (layer F.Cu) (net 3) (status 10))
 (segment (start 291.9816 -1059.32586) (end 284.15596 -1059.32586) (width 0.25) (layer F.Cu) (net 3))
 (segment (start 284.15596 -1059.32586) (end 278.0116 -1059.32586) (width 0.25) (layer F.Cu) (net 3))
 (segment (start 270.1916 -1059.32586) (end 270.2216 -1059.29586) (width 0.25) (layer F.Cu) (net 3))
 (segment (start 268.64174 -1059.40488) (end 268.67612 -1059.3705) (width 0.25) (layer F.Cu) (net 3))
 (segment (start 268.64174 -1062.84522) (end 268.64174 -1059.40488) (width 0.25) (layer F.Cu) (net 3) (status 10))
 (segment (start 264.0416 -1059.32586) (end 268.67612 -1059.3705) (width 0.25) (layer F.Cu) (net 3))
 (segment (start 268.67612 -1059.3705) (end 270.1916 -1059.32586) (width 0.25) (layer F.Cu) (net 3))
 (segment (start 260.25824 -1059.28922) (end 260.2616 -1059.28586) (width 0.25) (layer F.Cu) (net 3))
 (segment (start 255.66624 -1059.28922) (end 260.25824 -1059.28922) (width 0.25) (layer F.Cu) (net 3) (status 10))
 (segment (start 261.2436 -1051.74006) (end 261.2436 -1059.27954) (width 0.25) (layer F.Cu) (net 3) (status 10))
 (segment (start 261.2436 -1059.27954) (end 261.20598 -1059.31716) (width 0.25) (layer F.Cu) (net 3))
 (segment (start 264.0416 -1059.32586) (end 261.20598 -1059.31716) (width 0.25) (layer F.Cu) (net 3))
 (segment (start 261.20598 -1059.31716) (end 260.2616 -1059.28586) (width 0.25) (layer F.Cu) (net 3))
 (segment (start 299.3036 -1043.78006) (end 299.3636 -1043.72006) (width 0.25) (layer F.Cu) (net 1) (status 30))
 (segment (start 303.4936 -1043.72006) (end 303.6036 -1043.83006) (width 0.25) (layer F.Cu) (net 1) (status 30))
 (segment (start 299.3636 -1043.72006) (end 303.4936 -1043.72006) (width 0.25) (layer F.Cu) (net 1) (status 30))
 (segment (start 315.16828 -1062.83878) (end 315.15422 -1062.85284) (width 0.25) (layer F.Cu) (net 1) (status 30))
 (via (at 267.3858 -1060.49064) (size 0.8) (drill 0.4) (layers F.Cu B.Cu) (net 1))
 (segment (start 260.01218 -1060.49046) (end 267.38562 -1060.49046) (width 0.25) (layer F.Cu) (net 1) (status 10))
 (segment (start 267.38562 -1060.49046) (end 267.3858 -1060.49064) (width 0.25) (layer F.Cu) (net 1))
 (segment (start 267.3858 -1060.49064) (end 285.17596 -1060.49064) (width 0.25) (layer B.Cu) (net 1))
 (via (at 285.17596 -1060.49064) (size 0.8) (drill 0.4) (layers F.Cu B.Cu) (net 1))
 (via (at 300.9011 -1060.4754) (size 0.8) (drill 0.4) (layers F.Cu B.Cu) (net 1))
 (segment (start 285.17596 -1060.49064) (end 300.88586 -1060.49064) (width 0.25) (layer B.Cu) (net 1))
 (segment (start 300.88586 -1060.49064) (end 300.9011 -1060.4754) (width 0.25) (layer B.Cu) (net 1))
 (segment (start 300.9011 -1062.95072) (end 300.91752 -1062.96714) (width 0.25) (layer F.Cu) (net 1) (status 30))
 (segment (start 300.9011 -1060.4754) (end 300.9011 -1062.95072) (width 0.25) (layer F.Cu) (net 1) (status 20))
 (segment (start 285.17596 -1062.86944) (end 285.19492 -1062.8884) (width 0.25) (layer F.Cu) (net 1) (status 30))
 (segment (start 285.17596 -1060.49064) (end 285.17596 -1062.86944) (width 0.25) (layer F.Cu) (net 1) (status 20))
 (segment (start 300.9011 -1060.4754) (end 315.14542 -1060.4754) (width 0.25) (layer B.Cu) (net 1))
 (via (at 315.14542 -1060.4754) (size 0.8) (drill 0.4) (layers F.Cu B.Cu) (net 1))
 (segment (start 315.14542 -1062.84404) (end 315.15422 -1062.85284) (width 0.25) (layer F.Cu) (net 1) (status 30))
 (segment (start 315.14542 -1060.4754) (end 315.14542 -1062.84404) (width 0.25) (layer F.Cu) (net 1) (status 20))
 (segment (start 303.6036 -1052.81506) (end 305.84358 -1055.05504) (width 0.25) (layer F.Cu) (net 1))
 (segment (start 303.6036 -1051.79006) (end 303.6036 -1052.81506) (width 0.25) (layer F.Cu) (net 1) (status 10))
 (segment (start 309.72506 -1055.05504) (end 315.14542 -1060.4754) (width 0.25) (layer F.Cu) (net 1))
 (segment (start 305.84358 -1055.05504) (end 309.72506 -1055.05504) (width 0.25) (layer F.Cu) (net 1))
 (segment (start 265.8536 -1049.42006) (end 265.7936 -1049.48006) (width 0.25) (layer F.Cu) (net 4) (status 30))
 (segment (start 265.8536 -1045.86006) (end 265.8536 -1049.42006) (width 0.25) (layer F.Cu) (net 4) (status 30))
 (segment (start 299.3636 -1049.67006) (end 299.4336 -1049.74006) (width 0.25) (layer F.Cu) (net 2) (status 30))
 (segment (start 299.3636 -1045.92006) (end 299.3636 -1049.67006) (width 0.25) (layer F.Cu) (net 2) (status 30)))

